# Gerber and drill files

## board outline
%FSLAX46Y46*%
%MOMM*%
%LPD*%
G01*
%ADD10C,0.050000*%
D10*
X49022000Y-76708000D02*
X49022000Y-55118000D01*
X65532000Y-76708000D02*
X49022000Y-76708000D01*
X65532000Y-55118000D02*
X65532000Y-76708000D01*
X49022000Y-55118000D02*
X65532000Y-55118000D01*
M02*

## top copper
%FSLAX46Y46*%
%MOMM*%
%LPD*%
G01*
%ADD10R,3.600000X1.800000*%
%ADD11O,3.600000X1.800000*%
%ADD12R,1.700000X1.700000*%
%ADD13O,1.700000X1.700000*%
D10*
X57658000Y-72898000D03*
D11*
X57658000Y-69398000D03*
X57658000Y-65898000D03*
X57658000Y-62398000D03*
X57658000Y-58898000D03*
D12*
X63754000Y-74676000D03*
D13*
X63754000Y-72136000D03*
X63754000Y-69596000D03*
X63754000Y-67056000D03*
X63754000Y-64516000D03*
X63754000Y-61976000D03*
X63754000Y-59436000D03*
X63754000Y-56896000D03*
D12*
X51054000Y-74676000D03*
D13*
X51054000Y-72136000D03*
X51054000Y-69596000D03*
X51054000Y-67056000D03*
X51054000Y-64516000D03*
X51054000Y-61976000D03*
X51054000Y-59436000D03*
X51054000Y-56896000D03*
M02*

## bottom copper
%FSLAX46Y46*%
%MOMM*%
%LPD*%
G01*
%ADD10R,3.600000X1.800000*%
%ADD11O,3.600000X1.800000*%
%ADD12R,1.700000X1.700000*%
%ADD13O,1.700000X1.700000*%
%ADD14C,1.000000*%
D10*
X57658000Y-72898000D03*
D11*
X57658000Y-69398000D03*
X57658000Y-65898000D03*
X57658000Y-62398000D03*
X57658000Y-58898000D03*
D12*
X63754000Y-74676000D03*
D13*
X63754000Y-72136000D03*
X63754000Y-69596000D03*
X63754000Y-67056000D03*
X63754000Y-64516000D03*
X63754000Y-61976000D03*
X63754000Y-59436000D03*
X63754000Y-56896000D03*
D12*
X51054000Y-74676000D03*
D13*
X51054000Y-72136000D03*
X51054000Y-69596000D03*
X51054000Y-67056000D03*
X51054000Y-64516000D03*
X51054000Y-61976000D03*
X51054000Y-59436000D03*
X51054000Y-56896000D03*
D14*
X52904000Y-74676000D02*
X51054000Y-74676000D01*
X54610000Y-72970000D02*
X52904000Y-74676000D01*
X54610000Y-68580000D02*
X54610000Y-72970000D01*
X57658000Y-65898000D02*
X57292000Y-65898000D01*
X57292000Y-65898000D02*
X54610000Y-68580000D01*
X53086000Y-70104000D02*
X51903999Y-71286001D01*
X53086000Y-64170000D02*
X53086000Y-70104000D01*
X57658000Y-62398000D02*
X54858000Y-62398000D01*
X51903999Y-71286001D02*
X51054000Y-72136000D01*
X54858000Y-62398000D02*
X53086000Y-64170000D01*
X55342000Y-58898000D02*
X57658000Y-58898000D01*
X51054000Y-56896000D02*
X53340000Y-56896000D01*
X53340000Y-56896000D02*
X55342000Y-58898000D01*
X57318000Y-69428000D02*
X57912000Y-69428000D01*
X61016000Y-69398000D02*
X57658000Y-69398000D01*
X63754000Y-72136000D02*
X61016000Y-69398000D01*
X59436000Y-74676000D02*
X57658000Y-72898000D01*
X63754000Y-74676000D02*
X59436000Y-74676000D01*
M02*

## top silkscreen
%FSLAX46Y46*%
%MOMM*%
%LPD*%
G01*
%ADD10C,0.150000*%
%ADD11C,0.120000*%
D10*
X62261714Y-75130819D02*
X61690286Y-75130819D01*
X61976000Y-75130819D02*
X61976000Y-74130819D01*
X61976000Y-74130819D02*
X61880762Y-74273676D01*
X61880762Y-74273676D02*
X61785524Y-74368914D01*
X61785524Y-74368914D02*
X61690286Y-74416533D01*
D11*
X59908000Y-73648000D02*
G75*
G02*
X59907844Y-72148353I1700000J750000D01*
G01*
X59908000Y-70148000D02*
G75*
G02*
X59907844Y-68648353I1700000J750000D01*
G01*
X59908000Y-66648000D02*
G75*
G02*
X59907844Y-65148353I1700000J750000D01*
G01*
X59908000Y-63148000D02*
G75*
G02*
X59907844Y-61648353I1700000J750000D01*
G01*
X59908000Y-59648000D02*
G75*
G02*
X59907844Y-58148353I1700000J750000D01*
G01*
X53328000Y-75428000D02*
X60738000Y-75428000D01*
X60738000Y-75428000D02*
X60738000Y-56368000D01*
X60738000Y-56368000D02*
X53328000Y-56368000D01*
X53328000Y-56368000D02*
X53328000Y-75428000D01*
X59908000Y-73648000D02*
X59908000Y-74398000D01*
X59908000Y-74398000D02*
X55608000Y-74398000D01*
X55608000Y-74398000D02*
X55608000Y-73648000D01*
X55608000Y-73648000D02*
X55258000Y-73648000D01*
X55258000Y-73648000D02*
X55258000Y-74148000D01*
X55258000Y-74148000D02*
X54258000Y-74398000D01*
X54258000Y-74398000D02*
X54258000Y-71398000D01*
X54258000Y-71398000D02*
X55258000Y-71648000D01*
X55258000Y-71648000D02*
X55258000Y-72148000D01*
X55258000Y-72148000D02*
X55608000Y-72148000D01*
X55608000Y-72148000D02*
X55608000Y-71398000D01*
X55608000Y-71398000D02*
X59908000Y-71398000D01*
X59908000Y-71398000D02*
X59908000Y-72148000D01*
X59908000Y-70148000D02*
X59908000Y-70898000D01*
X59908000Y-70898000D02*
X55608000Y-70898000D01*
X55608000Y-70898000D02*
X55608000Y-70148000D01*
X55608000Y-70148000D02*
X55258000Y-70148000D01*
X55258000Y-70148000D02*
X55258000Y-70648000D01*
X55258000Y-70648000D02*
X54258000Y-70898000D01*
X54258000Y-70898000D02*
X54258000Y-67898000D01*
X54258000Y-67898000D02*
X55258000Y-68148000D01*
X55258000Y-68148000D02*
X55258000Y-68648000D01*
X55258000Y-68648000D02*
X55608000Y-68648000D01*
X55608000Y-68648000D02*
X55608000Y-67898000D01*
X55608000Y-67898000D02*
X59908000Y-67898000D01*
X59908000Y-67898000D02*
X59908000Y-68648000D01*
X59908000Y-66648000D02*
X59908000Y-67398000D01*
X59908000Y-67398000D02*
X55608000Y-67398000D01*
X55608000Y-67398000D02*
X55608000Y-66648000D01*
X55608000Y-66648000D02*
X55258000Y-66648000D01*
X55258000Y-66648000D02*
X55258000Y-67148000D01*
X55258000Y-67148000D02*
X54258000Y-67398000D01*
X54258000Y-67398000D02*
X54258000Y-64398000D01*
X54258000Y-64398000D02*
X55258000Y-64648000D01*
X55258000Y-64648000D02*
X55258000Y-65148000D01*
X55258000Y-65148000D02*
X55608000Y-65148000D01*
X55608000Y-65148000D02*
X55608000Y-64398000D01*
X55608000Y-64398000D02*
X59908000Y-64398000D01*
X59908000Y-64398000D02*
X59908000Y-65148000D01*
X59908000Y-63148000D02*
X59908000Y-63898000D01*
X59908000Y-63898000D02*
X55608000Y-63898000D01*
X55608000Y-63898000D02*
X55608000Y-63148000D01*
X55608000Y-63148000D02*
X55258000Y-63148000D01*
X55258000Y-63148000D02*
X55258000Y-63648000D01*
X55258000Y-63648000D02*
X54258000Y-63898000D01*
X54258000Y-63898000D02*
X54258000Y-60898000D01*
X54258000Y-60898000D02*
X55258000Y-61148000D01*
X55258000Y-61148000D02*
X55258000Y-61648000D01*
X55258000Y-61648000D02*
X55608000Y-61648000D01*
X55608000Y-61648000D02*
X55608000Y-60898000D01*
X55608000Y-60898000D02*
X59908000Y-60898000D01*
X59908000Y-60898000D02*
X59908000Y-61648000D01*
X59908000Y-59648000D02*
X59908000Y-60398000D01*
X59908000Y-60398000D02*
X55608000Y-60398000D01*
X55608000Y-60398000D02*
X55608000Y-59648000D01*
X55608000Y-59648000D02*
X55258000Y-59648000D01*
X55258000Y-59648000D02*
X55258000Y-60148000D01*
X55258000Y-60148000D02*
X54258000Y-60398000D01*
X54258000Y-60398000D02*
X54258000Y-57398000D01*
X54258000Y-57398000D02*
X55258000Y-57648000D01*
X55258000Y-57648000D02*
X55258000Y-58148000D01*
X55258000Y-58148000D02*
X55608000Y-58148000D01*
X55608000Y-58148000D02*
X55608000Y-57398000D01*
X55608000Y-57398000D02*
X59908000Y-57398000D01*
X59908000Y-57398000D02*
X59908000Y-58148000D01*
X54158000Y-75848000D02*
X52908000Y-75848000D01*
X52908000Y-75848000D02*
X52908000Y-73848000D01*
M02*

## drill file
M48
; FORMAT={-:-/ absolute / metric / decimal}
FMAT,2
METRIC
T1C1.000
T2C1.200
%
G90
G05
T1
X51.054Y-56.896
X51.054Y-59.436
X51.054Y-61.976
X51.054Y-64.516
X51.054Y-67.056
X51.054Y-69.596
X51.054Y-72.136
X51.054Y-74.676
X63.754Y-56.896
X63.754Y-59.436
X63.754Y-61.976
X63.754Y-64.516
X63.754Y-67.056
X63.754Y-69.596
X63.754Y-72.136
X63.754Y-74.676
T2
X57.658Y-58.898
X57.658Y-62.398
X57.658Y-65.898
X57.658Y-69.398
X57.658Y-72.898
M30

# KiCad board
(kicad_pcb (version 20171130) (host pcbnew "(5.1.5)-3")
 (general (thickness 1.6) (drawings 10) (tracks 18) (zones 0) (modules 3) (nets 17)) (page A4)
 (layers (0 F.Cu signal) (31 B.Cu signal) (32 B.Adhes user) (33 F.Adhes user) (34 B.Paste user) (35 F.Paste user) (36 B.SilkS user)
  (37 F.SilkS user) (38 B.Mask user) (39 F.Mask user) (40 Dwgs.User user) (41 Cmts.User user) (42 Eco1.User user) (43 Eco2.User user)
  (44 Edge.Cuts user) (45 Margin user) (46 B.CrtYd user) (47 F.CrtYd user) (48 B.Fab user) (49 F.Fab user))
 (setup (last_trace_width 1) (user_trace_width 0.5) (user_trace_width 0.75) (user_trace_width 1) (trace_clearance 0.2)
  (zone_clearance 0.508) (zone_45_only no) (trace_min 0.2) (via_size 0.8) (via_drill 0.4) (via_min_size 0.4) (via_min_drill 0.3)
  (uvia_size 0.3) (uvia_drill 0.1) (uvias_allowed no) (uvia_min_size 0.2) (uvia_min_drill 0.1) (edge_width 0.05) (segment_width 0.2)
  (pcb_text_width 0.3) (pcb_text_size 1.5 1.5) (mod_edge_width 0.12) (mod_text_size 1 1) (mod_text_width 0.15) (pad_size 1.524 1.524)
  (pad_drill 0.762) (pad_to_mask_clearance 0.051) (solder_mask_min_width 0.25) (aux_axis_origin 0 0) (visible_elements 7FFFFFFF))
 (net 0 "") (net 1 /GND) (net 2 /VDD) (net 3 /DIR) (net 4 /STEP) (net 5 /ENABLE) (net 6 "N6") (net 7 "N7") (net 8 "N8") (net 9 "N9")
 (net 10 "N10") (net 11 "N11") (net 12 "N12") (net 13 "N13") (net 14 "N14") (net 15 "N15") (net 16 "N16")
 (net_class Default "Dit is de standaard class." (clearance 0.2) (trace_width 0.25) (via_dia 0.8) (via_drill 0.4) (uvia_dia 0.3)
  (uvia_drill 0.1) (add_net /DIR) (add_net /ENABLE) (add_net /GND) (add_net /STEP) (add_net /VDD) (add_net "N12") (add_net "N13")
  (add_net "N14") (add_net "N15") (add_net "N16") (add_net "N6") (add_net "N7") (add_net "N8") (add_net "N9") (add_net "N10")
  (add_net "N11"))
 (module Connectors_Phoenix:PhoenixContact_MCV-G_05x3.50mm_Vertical (layer F.Cu) (at 57.658 72.898 90)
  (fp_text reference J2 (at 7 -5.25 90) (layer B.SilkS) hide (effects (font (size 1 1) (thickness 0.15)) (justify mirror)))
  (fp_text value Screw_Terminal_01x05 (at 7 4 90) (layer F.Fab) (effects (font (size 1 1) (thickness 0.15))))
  (fp_arc (start 0 3.95) (end -0.75 2.25) (angle 47.6) (layer F.SilkS) (width 0.12))
  (fp_arc (start 3.5 3.95) (end 2.75 2.25) (angle 47.6) (layer F.SilkS) (width 0.12))
  (fp_arc (start 7 3.95) (end 6.25 2.25) (angle 47.6) (layer F.SilkS) (width 0.12))
  (fp_arc (start 10.5 3.95) (end 9.75 2.25) (angle 47.6) (layer F.SilkS) (width 0.12))
  (fp_arc (start 14 3.95) (end 13.25 2.25) (angle 47.6) (layer F.SilkS) (width 0.12))
  (fp_line (start -2.53 -4.33) (end -2.53 3.08) (layer F.SilkS) (width 0.12))
  (fp_line (start -2.53 3.08) (end 16.53 3.08) (layer F.SilkS) (width 0.12))
  (fp_line (start 16.53 3.08) (end 16.53 -4.33) (layer F.SilkS) (width 0.12))
  (fp_line (start 16.53 -4.33) (end -2.53 -4.33) (layer F.SilkS) (width 0.12))
  (fp_line (start -0.75 2.25) (end -1.5 2.25) (layer F.SilkS) (width 0.12))
  (fp_line (start -1.5 2.25) (end -1.5 -2.05) (layer F.SilkS) (width 0.12))
  (fp_line (start -1.5 -2.05) (end -0.75 -2.05) (layer F.SilkS) (width 0.12))
  (fp_line (start -0.75 -2.05) (end -0.75 -2.4) (layer F.SilkS) (width 0.12))
  (fp_line (start -0.75 -2.4) (end -1.25 -2.4) (layer F.SilkS) (width 0.12))
  (fp_line (start -1.25 -2.4) (end -1.5 -3.4) (layer F.SilkS) (width 0.12))
  (fp_line (start -1.5 -3.4) (end 1.5 -3.4) (layer F.SilkS) (width 0.12))
  (fp_line (start 1.5 -3.4) (end 1.25 -2.4) (layer F.SilkS) (width 0.12))
  (fp_line (start 1.25 -2.4) (end 0.75 -2.4) (layer F.SilkS) (width 0.12))
  (fp_line (start 0.75 -2.4) (end 0.75 -2.05) (layer F.SilkS) (width 0.12))
  (fp_line (start 0.75 -2.05) (end 1.5 -2.05) (layer F.SilkS) (width 0.12))
  (fp_line (start 1.5 -2.05) (end 1.5 2.25) (layer F.SilkS) (width 0.12))
  (fp_line (start 1.5 2.25) (end 0.75 2.25) (layer F.SilkS) (width 0.12))
  (fp_line (start 2.75 2.25) (end 2 2.25) (layer F.SilkS) (width 0.12))
  (fp_line (start 2 2.25) (end 2 -2.05) (layer F.SilkS) (width 0.12))
  (fp_line (start 2 -2.05) (end 2.75 -2.05) (layer F.SilkS) (width 0.12))
  (fp_line (start 2.75 -2.05) (end 2.75 -2.4) (layer F.SilkS) (width 0.12))
  (fp_line (start 2.75 -2.4) (end 2.25 -2.4) (layer F.SilkS) (width 0.12))
  (fp_line (start 2.25 -2.4) (end 2 -3.4) (layer F.SilkS) (width 0.12))
  (fp_line (start 2 -3.4) (end 5 -3.4) (layer F.SilkS) (width 0.12))
  (fp_line (start 5 -3.4) (end 4.75 -2.4) (layer F.SilkS) (width 0.12))
  (fp_line (start 4.75 -2.4) (end 4.25 -2.4) (layer F.SilkS) (width 0.12))
  (fp_line (start 4.25 -2.4) (end 4.25 -2.05) (layer F.SilkS) (width 0.12))
  (fp_line (start 4.25 -2.05) (end 5 -2.05) (layer F.SilkS) (width 0.12))
  (fp_line (start 5 -2.05) (end 5 2.25) (layer F.SilkS) (width 0.12))
  (fp_line (start 5 2.25) (end 4.25 2.25) (layer F.SilkS) (width 0.12))
  (fp_line (start 6.25 2.25) (end 5.5 2.25) (layer F.SilkS) (width 0.12))
  (fp_line (start 5.5 2.25) (end 5.5 -2.05) (layer F.SilkS) (width 0.12))
  (fp_line (start 5.5 -2.05) (end 6.25 -2.05) (layer F.SilkS) (width 0.12))
  (fp_line (start 6.25 -2.05) (end 6.25 -2.4) (layer F.SilkS) (width 0.12))
  (fp_line (start 6.25 -2.4) (end 5.75 -2.4) (layer F.SilkS) (width 0.12))
  (fp_line (start 5.75 -2.4) (end 5.5 -3.4) (layer F.SilkS) (width 0.12))
  (fp_line (start 5.5 -3.4) (end 8.5 -3.4) (layer F.SilkS) (width 0.12))
  (fp_line (start 8.5 -3.4) (end 8.25 -2.4) (layer F.SilkS) (width 0.12))
  (fp_line (start 8.25 -2.4) (end 7.75 -2.4) (layer F.SilkS) (width 0.12))
  (fp_line (start 7.75 -2.4) (end 7.75 -2.05) (layer F.SilkS) (width 0.12))
  (fp_line (start 7.75 -2.05) (end 8.5 -2.05) (layer F.SilkS) (width 0.12))
  (fp_line (start 8.5 -2.05) (end 8.5 2.25) (layer F.SilkS) (width 0.12))
  (fp_line (start 8.5 2.25) (end 7.75 2.25) (layer F.SilkS) (width 0.12))
  (fp_line (start 9.75 2.25) (end 9 2.25) (layer F.SilkS) (width 0.12))
  (fp_line (start 9 2.25) (end 9 -2.05) (layer F.SilkS) (width 0.12))
  (fp_line (start 9 -2.05) (end 9.75 -2.05) (layer F.SilkS) (width 0.12))
  (fp_line (start 9.75 -2.05) (end 9.75 -2.4) (layer F.SilkS) (width 0.12))
  (fp_line (start 9.75 -2.4) (end 9.25 -2.4) (layer F.SilkS) (width 0.12))
  (fp_line (start 9.25 -2.4) (end 9 -3.4) (layer F.SilkS) (width 0.12))
  (fp_line (start 9 -3.4) (end 12 -3.4) (layer F.SilkS) (width 0.12))
  (fp_line (start 12 -3.4) (end 11.75 -2.4) (layer F.SilkS) (width 0.12))
  (fp_line (start 11.75 -2.4) (end 11.25 -2.4) (layer F.SilkS) (width 0.12))
  (fp_line (start 11.25 -2.4) (end 11.25 -2.05) (layer F.SilkS) (width 0.12))
  (fp_line (start 11.25 -2.05) (end 12 -2.05) (layer F.SilkS) (width 0.12))
  (fp_line (start 12 -2.05) (end 12 2.25) (layer F.SilkS) (width 0.12))
  (fp_line (start 12 2.25) (end 11.25 2.25) (layer F.SilkS) (width 0.12))
  (fp_line (start 13.25 2.25) (end 12.5 2.25) (layer F.SilkS) (width 0.12))
  (fp_line (start 12.5 2.25) (end 12.5 -2.05) (layer F.SilkS) (width 0.12))
  (fp_line (start 12.5 -2.05) (end 13.25 -2.05) (layer F.SilkS) (width 0.12))
  (fp_line (start 13.25 -2.05) (end 13.25 -2.4) (layer F.SilkS) (width 0.12))
  (fp_line (start 13.25 -2.4) (end 12.75 -2.4) (layer F.SilkS) (width 0.12))
  (fp_line (start 12.75 -2.4) (end 12.5 -3.4) (layer F.SilkS) (width 0.12))
  (fp_line (start 12.5 -3.4) (end 15.5 -3.4) (layer F.SilkS) (width 0.12))
  (fp_line (start 15.5 -3.4) (end 15.25 -2.4) (layer F.SilkS) (width 0.12))
  (fp_line (start 15.25 -2.4) (end 14.75 -2.4) (layer F.SilkS) (width 0.12))
  (fp_line (start 14.75 -2.4) (end 14.75 -2.05) (layer F.SilkS) (width 0.12))
  (fp_line (start 14.75 -2.05) (end 15.5 -2.05) (layer F.SilkS) (width 0.12))
  (fp_line (start 15.5 -2.05) (end 15.5 2.25) (layer F.SilkS) (width 0.12))
  (fp_line (start 15.5 2.25) (end 14.75 2.25) (layer F.SilkS) (width 0.12))
  (fp_line (start -2.95 -3.5) (end -2.95 -4.75) (layer F.SilkS) (width 0.12))
  (fp_line (start -2.95 -4.75) (end -0.95 -4.75) (layer F.SilkS) (width 0.12))
  (pad 1 thru_hole rect (at 0 0 90) (size 1.8 3.6) (drill 1.2) (layers *.Cu *.Mask) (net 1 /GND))
  (pad 2 thru_hole oval (at 3.5 0 90) (size 1.8 3.6) (drill 1.2) (layers *.Cu *.Mask) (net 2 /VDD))
  (pad 3 thru_hole oval (at 7 0 90) (size 1.8 3.6) (drill 1.2) (layers *.Cu *.Mask) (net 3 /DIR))
  (pad 4 thru_hole oval (at 10.5 0 90) (size 1.8 3.6) (drill 1.2) (layers *.Cu *.Mask) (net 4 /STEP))
  (pad 5 thru_hole oval (at 14 0 90) (size 1.8 3.6) (drill 1.2) (layers *.Cu *.Mask) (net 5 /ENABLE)))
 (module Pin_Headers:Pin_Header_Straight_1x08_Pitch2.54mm (layer B.Cu) (at 63.754 74.676)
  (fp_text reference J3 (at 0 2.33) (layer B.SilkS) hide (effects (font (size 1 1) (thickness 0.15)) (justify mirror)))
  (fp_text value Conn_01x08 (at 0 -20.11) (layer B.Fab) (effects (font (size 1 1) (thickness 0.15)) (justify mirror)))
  (pad 1 thru_hole rect (at 0 0) (size 1.7 1.7) (drill 1) (layers *.Cu *.Mask) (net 1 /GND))
  (pad 2 thru_hole oval (at 0 -2.54) (size 1.7 1.7) (drill 1) (layers *.Cu *.Mask) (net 2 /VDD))
  (pad 3 thru_hole oval (at 0 -5.08) (size 1.7 1.7) (drill 1) (layers *.Cu *.Mask) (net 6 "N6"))
  (pad 4 thru_hole oval (at 0 -7.62) (size 1.7 1.7) (drill 1) (layers *.Cu *.Mask) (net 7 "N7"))
  (pad 5 thru_hole oval (at 0 -10.16) (size 1.7 1.7) (drill 1) (layers *.Cu *.Mask) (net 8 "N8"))
  (pad 6 thru_hole oval (at 0 -12.7) (size 1.7 1.7) (drill 1) (layers *.Cu *.Mask) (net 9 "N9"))
  (pad 7 thru_hole oval (at 0 -15.24) (size 1.7 1.7) (drill 1) (layers *.Cu *.Mask) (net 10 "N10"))
  (pad 8 thru_hole oval (at 0 -17.78) (size 1.7 1.7) (drill 1) (layers *.Cu *.Mask) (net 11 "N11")))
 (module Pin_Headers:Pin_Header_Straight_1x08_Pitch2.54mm (layer B.Cu) (at 51.054 74.676)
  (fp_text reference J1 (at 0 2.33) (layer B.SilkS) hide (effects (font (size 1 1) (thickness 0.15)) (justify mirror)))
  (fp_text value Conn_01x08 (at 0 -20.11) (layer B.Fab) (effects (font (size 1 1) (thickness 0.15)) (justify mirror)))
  (pad 1 thru_hole rect (at 0 0) (size 1.7 1.7) (drill 1) (layers *.Cu *.Mask) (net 3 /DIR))
  (pad 2 thru_hole oval (at 0 -2.54) (size 1.7 1.7) (drill 1) (layers *.Cu *.Mask) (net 4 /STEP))
  (pad 3 thru_hole oval (at 0 -5.08) (size 1.7 1.7) (drill 1) (layers *.Cu *.Mask) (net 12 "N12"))
  (pad 4 thru_hole oval (at 0 -7.62) (size 1.7 1.7) (drill 1) (layers *.Cu *.Mask) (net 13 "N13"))
  (pad 5 thru_hole oval (at 0 -10.16) (size 1.7 1.7) (drill 1) (layers *.Cu *.Mask) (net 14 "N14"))
  (pad 6 thru_hole oval (at 0 -12.7) (size 1.7 1.7) (drill 1) (layers *.Cu *.Mask) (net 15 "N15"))
  (pad 7 thru_hole oval (at 0 -15.24) (size 1.7 1.7) (drill 1) (layers *.Cu *.Mask) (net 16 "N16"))
  (pad 8 thru_hole oval (at 0 -17.78) (size 1.7 1.7) (drill 1) (layers *.Cu *.Mask) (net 5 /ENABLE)))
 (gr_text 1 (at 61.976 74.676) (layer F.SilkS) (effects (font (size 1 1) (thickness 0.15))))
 (gr_line (start 49.022 76.708) (end 49.022 55.118) (layer Edge.Cuts) (width 0.05))
 (gr_line (start 65.532 76.708) (end 49.022 76.708) (layer Edge.Cuts) (width 0.05))
 (gr_line (start 65.532 55.118) (end 65.532 76.708) (layer Edge.Cuts) (width 0.05))
 (gr_line (start 49.022 55.118) (end 65.532 55.118) (layer Edge.Cuts) (width 0.05))
 (segment (start 52.904 74.676) (end 51.054 74.676) (width 1) (layer B.Cu) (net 3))
 (segment (start 54.61 72.97) (end 52.904 74.676) (width 1) (layer B.Cu) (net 3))
 (segment (start 54.61 68.58) (end 54.61 72.97) (width 1) (layer B.Cu) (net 3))
 (segment (start 57.658 65.898) (end 57.292 65.898) (width 1) (layer B.Cu) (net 3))
 (segment (start 57.292 65.898) (end 54.61 68.58) (width 1) (layer B.Cu) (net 3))
 (segment (start 53.086 70.104) (end 51.903999 71.286001) (width 1) (layer B.Cu) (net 4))
 (segment (start 53.086 64.17) (end 53.086 70.104) (width 1) (layer B.Cu) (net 4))
 (segment (start 57.658 62.398) (end 54.858 62.398) (width 1) (layer B.Cu) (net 4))
 (segment (start 51.903999 71.286001) (end 51.054 72.136) (width 1) (layer B.Cu) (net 4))
 (segment (start 54.858 62.398) (end 53.086 64.17) (width 1) (layer B.Cu) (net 4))
 (segment (start 55.342 58.898) (end 57.658 58.898) (width 1) (layer B.Cu) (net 5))
 (segment (start 51.054 56.896) (end 53.34 56.896) (width 1) (layer B.Cu) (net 5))
 (segment (start 53.34 56.896) (end 55.342 58.898) (width 1) (layer B.Cu) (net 5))
 (segment (start 57.318 69.428) (end 57.912 69.428) (width 1) (layer B.Cu) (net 2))
 (segment (start 61.016 69.398) (end 57.658 69.398) (width 1) (layer B.Cu) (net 2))
 (segment (start 63.754 72.136) (end 61.016 69.398) (width 1) (layer B.Cu) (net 2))
 (segment (start 59.436 74.676) (end 57.658 72.898) (width 1) (layer B.Cu) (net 1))
 (segment (start 63.754 74.676) (end 59.436 74.676) (width 1) (layer B.Cu) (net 1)))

